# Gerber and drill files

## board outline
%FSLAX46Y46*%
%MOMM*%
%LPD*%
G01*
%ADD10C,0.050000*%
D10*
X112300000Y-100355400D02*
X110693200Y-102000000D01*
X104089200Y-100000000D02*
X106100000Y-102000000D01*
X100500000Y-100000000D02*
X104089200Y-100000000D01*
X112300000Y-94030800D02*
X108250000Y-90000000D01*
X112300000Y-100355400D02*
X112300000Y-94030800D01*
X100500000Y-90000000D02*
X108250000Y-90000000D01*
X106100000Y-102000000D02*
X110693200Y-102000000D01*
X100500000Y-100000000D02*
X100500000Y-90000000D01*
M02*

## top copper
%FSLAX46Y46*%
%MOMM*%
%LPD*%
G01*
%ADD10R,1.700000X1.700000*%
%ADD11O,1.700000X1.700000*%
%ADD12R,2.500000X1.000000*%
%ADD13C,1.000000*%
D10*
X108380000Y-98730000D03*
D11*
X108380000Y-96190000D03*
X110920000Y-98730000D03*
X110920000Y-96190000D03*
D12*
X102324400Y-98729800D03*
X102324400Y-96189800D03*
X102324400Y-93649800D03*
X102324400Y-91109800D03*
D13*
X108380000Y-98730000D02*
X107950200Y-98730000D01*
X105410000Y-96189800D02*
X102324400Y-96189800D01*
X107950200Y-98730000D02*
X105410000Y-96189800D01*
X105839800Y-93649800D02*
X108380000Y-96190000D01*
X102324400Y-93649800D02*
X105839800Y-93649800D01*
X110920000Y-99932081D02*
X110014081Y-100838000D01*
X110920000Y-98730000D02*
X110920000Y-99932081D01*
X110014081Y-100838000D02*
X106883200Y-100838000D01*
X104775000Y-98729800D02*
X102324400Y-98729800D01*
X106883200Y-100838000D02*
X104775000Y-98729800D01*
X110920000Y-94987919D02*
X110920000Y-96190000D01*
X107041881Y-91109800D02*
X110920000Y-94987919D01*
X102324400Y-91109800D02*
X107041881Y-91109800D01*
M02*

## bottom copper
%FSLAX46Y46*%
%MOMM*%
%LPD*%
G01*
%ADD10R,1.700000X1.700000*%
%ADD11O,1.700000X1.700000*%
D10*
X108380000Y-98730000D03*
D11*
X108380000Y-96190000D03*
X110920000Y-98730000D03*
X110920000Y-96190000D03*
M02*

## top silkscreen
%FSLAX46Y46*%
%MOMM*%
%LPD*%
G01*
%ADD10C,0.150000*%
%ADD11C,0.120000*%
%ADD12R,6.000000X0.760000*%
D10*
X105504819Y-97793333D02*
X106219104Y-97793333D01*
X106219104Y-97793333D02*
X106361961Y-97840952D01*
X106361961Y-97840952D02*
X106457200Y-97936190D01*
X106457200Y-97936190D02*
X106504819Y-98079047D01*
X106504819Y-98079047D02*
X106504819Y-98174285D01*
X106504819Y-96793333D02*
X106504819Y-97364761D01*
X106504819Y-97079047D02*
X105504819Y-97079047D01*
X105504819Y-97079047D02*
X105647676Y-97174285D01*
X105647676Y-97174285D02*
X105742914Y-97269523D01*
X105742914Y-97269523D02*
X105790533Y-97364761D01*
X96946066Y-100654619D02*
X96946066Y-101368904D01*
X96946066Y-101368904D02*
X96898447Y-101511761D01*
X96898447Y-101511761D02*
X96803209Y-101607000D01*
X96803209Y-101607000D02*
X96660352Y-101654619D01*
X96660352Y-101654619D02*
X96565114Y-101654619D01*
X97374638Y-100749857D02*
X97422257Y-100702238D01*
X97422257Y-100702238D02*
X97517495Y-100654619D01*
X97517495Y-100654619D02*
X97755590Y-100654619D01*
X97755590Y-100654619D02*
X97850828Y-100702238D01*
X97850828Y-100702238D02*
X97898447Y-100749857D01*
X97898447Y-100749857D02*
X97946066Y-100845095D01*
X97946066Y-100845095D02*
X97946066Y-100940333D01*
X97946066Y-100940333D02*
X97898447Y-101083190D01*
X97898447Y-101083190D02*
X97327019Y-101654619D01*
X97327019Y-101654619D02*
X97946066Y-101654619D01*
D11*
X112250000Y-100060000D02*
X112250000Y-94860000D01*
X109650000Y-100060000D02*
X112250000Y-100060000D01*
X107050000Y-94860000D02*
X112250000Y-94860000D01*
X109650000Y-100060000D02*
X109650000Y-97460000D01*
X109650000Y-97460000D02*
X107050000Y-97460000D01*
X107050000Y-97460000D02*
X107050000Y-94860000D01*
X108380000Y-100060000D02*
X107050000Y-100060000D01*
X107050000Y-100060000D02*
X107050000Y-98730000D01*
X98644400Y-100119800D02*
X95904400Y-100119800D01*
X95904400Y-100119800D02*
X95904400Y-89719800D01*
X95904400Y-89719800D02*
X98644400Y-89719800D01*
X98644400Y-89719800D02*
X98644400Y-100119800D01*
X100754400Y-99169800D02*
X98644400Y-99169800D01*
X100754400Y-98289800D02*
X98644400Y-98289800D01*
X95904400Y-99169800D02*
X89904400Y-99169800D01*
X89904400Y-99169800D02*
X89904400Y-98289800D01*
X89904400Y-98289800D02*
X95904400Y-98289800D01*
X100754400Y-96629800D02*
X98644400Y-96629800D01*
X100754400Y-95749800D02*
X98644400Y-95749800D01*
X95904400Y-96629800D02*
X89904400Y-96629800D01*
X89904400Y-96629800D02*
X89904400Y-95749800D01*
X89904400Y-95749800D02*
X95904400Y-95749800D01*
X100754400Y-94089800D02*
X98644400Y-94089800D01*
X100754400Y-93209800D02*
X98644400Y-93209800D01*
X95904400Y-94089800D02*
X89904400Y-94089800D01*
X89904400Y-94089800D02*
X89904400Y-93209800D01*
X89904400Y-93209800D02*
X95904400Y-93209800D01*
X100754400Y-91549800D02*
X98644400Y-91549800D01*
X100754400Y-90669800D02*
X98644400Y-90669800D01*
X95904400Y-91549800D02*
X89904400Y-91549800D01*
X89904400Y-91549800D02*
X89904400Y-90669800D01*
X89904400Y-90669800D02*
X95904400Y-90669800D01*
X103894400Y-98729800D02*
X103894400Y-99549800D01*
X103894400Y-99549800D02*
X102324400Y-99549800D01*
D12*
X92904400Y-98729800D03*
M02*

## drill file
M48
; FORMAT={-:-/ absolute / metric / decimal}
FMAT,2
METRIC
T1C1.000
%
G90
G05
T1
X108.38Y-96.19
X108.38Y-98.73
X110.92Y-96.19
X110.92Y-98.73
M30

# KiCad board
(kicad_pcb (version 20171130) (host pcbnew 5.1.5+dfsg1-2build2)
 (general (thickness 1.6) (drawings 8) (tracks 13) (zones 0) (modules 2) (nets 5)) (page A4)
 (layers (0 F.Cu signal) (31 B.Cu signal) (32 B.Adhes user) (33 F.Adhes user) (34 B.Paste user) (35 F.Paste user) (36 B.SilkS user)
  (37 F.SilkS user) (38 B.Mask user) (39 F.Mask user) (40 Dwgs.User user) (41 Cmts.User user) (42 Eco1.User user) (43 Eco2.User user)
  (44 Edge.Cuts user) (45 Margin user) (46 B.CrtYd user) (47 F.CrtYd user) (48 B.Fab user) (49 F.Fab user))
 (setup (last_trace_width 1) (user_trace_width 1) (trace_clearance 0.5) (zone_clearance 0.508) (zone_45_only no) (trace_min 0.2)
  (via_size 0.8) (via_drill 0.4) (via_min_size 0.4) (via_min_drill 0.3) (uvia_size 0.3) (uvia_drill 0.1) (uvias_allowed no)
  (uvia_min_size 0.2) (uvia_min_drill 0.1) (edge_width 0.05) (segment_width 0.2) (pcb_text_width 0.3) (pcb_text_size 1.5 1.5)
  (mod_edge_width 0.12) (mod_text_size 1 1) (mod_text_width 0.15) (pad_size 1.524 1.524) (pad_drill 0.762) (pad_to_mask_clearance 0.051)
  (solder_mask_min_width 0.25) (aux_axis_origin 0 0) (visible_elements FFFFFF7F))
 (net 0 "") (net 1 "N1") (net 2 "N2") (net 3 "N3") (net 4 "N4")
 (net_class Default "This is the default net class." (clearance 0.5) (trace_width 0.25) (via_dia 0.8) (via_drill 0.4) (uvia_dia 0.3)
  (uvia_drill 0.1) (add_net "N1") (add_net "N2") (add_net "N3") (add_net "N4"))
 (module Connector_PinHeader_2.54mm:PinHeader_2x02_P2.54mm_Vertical (layer F.Cu) (at 108.38 98.73 90)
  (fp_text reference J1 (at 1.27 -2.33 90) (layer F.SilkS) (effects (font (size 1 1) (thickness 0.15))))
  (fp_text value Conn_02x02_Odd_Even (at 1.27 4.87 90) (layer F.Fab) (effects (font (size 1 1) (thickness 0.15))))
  (fp_line (start -1.33 3.87) (end 3.87 3.87) (layer F.SilkS) (width 0.12))
  (fp_line (start -1.33 1.27) (end -1.33 3.87) (layer F.SilkS) (width 0.12))
  (fp_line (start 3.87 -1.33) (end 3.87 3.87) (layer F.SilkS) (width 0.12))
  (fp_line (start -1.33 1.27) (end 1.27 1.27) (layer F.SilkS) (width 0.12))
  (fp_line (start 1.27 1.27) (end 1.27 -1.33) (layer F.SilkS) (width 0.12))
  (fp_line (start 1.27 -1.33) (end 3.87 -1.33) (layer F.SilkS) (width 0.12))
  (fp_line (start -1.33 0) (end -1.33 -1.33) (layer F.SilkS) (width 0.12))
  (fp_line (start -1.33 -1.33) (end 0 -1.33) (layer F.SilkS) (width 0.12))
  (pad 1 thru_hole rect (at 0 0 90) (size 1.7 1.7) (drill 1) (layers *.Cu *.Mask) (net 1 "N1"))
  (pad 2 thru_hole oval (at 2.54 0 90) (size 1.7 1.7) (drill 1) (layers *.Cu *.Mask) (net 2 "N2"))
  (pad 3 thru_hole oval (at 0 2.54 90) (size 1.7 1.7) (drill 1) (layers *.Cu *.Mask) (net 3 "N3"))
  (pad 4 thru_hole oval (at 2.54 2.54 90) (size 1.7 1.7) (drill 1) (layers *.Cu *.Mask) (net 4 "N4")))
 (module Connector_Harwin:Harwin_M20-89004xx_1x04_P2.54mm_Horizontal (layer F.Cu) (at 96.7994 94.9198 180)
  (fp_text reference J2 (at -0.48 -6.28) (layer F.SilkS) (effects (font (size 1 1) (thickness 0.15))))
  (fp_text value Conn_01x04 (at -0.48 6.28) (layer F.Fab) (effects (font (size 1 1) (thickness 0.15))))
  (fp_line (start -1.845 -5.2) (end 0.895 -5.2) (layer F.SilkS) (width 0.12))
  (fp_line (start 0.895 -5.2) (end 0.895 5.2) (layer F.SilkS) (width 0.12))
  (fp_line (start 0.895 5.2) (end -1.845 5.2) (layer F.SilkS) (width 0.12))
  (fp_line (start -1.845 5.2) (end -1.845 -5.2) (layer F.SilkS) (width 0.12))
  (fp_line (start -3.955 -4.25) (end -1.845 -4.25) (layer F.SilkS) (width 0.12))
  (fp_line (start -3.955 -3.37) (end -1.845 -3.37) (layer F.SilkS) (width 0.12))
  (fp_line (start 0.895 -4.25) (end 6.895 -4.25) (layer F.SilkS) (width 0.12))
  (fp_line (start 6.895 -4.25) (end 6.895 -3.37) (layer F.SilkS) (width 0.12))
  (fp_line (start 6.895 -3.37) (end 0.895 -3.37) (layer F.SilkS) (width 0.12))
  (fp_line (start -3.955 -1.71) (end -1.845 -1.71) (layer F.SilkS) (width 0.12))
  (fp_line (start -3.955 -0.83) (end -1.845 -0.83) (layer F.SilkS) (width 0.12))
  (fp_line (start 0.895 -1.71) (end 6.895 -1.71) (layer F.SilkS) (width 0.12))
  (fp_line (start 6.895 -1.71) (end 6.895 -0.83) (layer F.SilkS) (width 0.12))
  (fp_line (start 6.895 -0.83) (end 0.895 -0.83) (layer F.SilkS) (width 0.12))
  (fp_line (start -3.955 0.83) (end -1.845 0.83) (layer F.SilkS) (width 0.12))
  (fp_line (start -3.955 1.71) (end -1.845 1.71) (layer F.SilkS) (width 0.12))
  (fp_line (start 0.895 0.83) (end 6.895 0.83) (layer F.SilkS) (width 0.12))
  (fp_line (start 6.895 0.83) (end 6.895 1.71) (layer F.SilkS) (width 0.12))
  (fp_line (start 6.895 1.71) (end 0.895 1.71) (layer F.SilkS) (width 0.12))
  (fp_line (start -3.955 3.37) (end -1.845 3.37) (layer F.SilkS) (width 0.12))
  (fp_line (start -3.955 4.25) (end -1.845 4.25) (layer F.SilkS) (width 0.12))
  (fp_line (start 0.895 3.37) (end 6.895 3.37) (layer F.SilkS) (width 0.12))
  (fp_line (start 6.895 3.37) (end 6.895 4.25) (layer F.SilkS) (width 0.12))
  (fp_line (start 6.895 4.25) (end 0.895 4.25) (layer F.SilkS) (width 0.12))
  (fp_line (start -7.095 -3.81) (end -7.095 -4.63) (layer F.SilkS) (width 0.12))
  (fp_line (start -7.095 -4.63) (end -5.525 -4.63) (layer F.SilkS) (width 0.12))
  (pad 1 smd rect (at -5.525 -3.81 180) (size 2.5 1) (layers F.Cu F.Paste F.Mask) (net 3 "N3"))
  (pad 2 smd rect (at -5.525 -1.27 180) (size 2.5 1) (layers F.Cu F.Paste F.Mask) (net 1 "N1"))
  (pad 3 smd rect (at -5.525 1.27 180) (size 2.5 1) (layers F.Cu F.Paste F.Mask) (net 2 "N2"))
  (pad 4 smd rect (at -5.525 3.81 180) (size 2.5 1) (layers F.Cu F.Paste F.Mask) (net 4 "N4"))
  (pad "" smd rect (at 3.895 -3.81 180) (size 6 0.76) (layers F.SilkS)))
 (gr_line (start 112.3 100.3554) (end 110.6932 102) (layer Edge.Cuts) (width 0.05))
 (gr_line (start 104.0892 100) (end 106.1 102) (layer Edge.Cuts) (width 0.05))
 (gr_line (start 100.5 100) (end 104.0892 100) (layer Edge.Cuts) (width 0.05))
 (gr_line (start 112.3 94.0308) (end 108.25 90) (layer Edge.Cuts) (width 0.05))
 (gr_line (start 112.3 100.3554) (end 112.3 94.0308) (layer Edge.Cuts) (width 0.05))
 (gr_line (start 100.5 90) (end 108.25 90) (layer Edge.Cuts) (width 0.05))
 (gr_line (start 106.1 102) (end 110.6932 102) (layer Edge.Cuts) (width 0.05))
 (gr_line (start 100.5 100) (end 100.5 90) (layer Edge.Cuts) (width 0.05))
 (segment (start 108.38 98.73) (end 107.9502 98.73) (width 1) (layer F.Cu) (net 1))
 (segment (start 105.41 96.1898) (end 102.3244 96.1898) (width 1) (layer F.Cu) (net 1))
 (segment (start 107.9502 98.73) (end 105.41 96.1898) (width 1) (layer F.Cu) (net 1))
 (segment (start 105.8398 93.6498) (end 108.38 96.19) (width 1) (layer F.Cu) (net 2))
 (segment (start 102.3244 93.6498) (end 105.8398 93.6498) (width 1) (layer F.Cu) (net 2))
 (segment (start 110.92 99.932081) (end 110.014081 100.838) (width 1) (layer F.Cu) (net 3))
 (segment (start 110.92 98.73) (end 110.92 99.932081) (width 1) (layer F.Cu) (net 3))
 (segment (start 110.014081 100.838) (end 106.8832 100.838) (width 1) (layer F.Cu) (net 3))
 (segment (start 104.775 98.7298) (end 102.3244 98.7298) (width 1) (layer F.Cu) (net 3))
 (segment (start 106.8832 100.838) (end 104.775 98.7298) (width 1) (layer F.Cu) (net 3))
 (segment (start 110.92 94.987919) (end 110.92 96.19) (width 1) (layer F.Cu) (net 4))
 (segment (start 107.041881 91.1098) (end 110.92 94.987919) (width 1) (layer F.Cu) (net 4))
 (segment (start 102.3244 91.1098) (end 107.041881 91.1098) (width 1) (layer F.Cu) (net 4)))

